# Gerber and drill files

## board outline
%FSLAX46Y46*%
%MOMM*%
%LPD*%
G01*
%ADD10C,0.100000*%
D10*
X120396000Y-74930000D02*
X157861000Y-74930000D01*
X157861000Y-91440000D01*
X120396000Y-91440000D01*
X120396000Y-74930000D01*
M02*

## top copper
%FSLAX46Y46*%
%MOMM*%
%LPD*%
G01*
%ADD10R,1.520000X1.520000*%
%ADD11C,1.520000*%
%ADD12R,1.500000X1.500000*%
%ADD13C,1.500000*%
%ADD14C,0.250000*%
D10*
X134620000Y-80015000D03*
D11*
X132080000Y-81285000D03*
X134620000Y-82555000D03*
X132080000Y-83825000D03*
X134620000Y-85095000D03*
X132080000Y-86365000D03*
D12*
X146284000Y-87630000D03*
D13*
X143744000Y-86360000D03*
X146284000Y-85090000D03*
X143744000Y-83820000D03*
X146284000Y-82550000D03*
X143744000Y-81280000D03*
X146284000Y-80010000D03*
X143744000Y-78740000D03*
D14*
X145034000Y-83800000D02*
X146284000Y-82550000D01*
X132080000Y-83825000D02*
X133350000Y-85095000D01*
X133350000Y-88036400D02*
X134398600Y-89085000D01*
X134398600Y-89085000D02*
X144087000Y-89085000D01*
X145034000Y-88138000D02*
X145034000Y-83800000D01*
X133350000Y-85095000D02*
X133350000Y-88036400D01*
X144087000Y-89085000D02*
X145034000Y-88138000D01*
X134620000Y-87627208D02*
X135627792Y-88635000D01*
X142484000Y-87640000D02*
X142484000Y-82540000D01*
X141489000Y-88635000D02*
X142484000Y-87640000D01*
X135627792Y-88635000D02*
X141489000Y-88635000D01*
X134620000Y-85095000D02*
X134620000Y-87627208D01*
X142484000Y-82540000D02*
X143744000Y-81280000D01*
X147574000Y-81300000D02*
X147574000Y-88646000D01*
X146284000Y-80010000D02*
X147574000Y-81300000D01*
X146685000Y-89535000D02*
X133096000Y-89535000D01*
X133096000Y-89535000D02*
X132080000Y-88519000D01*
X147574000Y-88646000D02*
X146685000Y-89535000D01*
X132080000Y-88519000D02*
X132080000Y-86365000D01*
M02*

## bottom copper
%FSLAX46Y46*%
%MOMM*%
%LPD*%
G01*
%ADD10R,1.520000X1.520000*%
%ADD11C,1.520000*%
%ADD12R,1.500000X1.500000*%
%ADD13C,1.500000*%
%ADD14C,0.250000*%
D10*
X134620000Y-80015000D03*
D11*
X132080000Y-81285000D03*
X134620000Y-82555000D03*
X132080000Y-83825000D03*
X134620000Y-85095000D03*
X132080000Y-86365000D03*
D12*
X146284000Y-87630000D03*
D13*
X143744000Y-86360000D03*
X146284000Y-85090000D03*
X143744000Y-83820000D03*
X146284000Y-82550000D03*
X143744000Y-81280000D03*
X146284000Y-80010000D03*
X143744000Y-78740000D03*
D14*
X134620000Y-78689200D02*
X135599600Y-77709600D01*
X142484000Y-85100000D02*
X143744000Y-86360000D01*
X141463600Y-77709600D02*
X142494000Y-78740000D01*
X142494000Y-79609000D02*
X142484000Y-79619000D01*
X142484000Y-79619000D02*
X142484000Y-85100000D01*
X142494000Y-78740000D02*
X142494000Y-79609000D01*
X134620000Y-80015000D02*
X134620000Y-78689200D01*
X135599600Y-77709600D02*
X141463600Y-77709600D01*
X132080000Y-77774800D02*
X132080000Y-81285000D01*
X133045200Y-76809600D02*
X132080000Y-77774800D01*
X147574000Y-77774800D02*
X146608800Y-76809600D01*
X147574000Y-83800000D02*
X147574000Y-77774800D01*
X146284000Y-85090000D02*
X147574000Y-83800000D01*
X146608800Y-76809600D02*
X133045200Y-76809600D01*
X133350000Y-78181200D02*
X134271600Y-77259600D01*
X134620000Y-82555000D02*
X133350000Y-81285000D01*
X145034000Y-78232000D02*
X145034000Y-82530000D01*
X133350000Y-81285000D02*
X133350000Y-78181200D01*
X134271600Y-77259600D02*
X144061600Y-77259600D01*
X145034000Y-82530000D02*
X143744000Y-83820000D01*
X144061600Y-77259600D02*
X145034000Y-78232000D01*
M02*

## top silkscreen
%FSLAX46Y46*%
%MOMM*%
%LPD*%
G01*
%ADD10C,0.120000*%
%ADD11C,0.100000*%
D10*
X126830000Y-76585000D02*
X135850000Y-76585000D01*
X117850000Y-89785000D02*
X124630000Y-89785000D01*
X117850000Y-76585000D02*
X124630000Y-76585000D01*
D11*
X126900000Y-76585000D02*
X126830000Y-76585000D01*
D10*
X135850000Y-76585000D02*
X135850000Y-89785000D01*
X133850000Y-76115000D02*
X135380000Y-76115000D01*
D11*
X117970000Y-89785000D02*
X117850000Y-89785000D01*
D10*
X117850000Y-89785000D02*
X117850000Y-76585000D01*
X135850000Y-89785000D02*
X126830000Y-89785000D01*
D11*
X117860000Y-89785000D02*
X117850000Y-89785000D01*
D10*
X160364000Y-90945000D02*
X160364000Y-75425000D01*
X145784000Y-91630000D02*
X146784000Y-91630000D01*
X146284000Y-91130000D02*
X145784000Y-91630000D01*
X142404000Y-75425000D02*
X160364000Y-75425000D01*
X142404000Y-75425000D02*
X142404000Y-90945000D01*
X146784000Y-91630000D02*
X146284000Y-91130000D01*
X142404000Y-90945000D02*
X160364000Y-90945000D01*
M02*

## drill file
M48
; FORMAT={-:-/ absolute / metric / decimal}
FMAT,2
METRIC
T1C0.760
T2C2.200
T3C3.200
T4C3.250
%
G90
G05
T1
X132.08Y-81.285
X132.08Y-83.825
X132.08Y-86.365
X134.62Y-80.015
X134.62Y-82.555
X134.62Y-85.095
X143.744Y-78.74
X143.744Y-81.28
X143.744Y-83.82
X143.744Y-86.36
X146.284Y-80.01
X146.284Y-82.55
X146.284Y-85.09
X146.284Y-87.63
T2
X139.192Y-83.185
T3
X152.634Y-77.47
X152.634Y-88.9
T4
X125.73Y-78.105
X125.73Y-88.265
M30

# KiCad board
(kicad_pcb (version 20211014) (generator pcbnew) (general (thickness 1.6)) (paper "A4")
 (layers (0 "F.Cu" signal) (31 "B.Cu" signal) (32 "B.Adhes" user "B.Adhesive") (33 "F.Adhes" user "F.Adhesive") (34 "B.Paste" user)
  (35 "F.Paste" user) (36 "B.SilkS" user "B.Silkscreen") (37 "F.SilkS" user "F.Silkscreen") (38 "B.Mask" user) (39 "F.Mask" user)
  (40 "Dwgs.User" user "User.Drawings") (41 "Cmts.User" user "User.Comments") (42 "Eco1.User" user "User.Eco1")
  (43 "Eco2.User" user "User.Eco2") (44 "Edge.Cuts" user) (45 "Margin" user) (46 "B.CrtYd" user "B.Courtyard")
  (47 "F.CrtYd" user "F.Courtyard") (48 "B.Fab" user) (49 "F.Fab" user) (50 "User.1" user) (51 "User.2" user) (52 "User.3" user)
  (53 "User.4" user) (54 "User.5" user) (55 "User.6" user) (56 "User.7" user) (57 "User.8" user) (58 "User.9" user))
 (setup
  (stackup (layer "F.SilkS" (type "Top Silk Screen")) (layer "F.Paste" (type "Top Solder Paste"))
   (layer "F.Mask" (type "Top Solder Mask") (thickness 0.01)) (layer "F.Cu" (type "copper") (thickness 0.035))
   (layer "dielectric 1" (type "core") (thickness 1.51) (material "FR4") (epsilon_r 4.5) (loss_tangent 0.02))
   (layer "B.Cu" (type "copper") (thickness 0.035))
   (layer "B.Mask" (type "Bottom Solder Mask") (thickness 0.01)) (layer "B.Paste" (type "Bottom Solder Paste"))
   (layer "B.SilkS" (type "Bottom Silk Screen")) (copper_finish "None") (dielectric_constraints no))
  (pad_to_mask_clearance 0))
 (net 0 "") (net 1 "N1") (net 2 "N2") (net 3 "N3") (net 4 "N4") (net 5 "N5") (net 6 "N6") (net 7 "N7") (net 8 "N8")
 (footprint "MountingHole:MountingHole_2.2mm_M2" (layer "F.Cu") (at 139.192 83.185)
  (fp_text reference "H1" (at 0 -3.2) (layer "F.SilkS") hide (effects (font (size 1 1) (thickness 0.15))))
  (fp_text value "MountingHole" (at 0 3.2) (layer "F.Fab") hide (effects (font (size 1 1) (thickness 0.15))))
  (pad "" np_thru_hole circle (at 0 0) (size 2.2 2.2) (drill 2.2) (layers *.Cu *.Mask)))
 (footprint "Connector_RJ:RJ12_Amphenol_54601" (layer "F.Cu") (at 134.62 80.015 -90)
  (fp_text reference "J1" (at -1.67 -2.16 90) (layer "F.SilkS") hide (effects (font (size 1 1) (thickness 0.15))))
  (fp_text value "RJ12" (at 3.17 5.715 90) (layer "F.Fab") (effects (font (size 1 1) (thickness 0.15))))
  (fp_line (start -3.43 7.79) (end -3.43 -1.23) (layer "F.SilkS") (width 0.12))
  (fp_line (start 9.77 16.77) (end 9.77 9.99) (layer "F.SilkS") (width 0.12))
  (fp_line (start -3.43 16.77) (end -3.43 9.99) (layer "F.SilkS") (width 0.12))
  (fp_line (start -3.43 7.72) (end -3.43 7.79) (layer "F.SilkS") (width 0.1))
  (fp_line (start -3.43 -1.23) (end 9.77 -1.23) (layer "F.SilkS") (width 0.12))
  (fp_line (start -3.9 0.77) (end -3.9 -0.76) (layer "F.SilkS") (width 0.12))
  (fp_line (start 9.77 16.65) (end 9.77 16.77) (layer "F.SilkS") (width 0.1))
  (fp_line (start 9.77 16.77) (end -3.43 16.77) (layer "F.SilkS") (width 0.12))
  (fp_line (start 9.77 -1.23) (end 9.77 7.79) (layer "F.SilkS") (width 0.12))
  (fp_line (start 9.77 16.76) (end 9.77 16.77) (layer "F.SilkS") (width 0.1))
  (pad "" np_thru_hole circle (at 8.25 8.89 270) (size 3.25 3.25) (drill 3.25) (layers *.Cu *.Mask))
  (pad "" np_thru_hole circle (at -1.91 8.89 270) (size 3.25 3.25) (drill 3.25) (layers *.Cu *.Mask))
  (pad "1" thru_hole rect (at 0 0 270) (size 1.52 1.52) (drill 0.76) (layers *.Cu *.Mask) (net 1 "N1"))
  (pad "2" thru_hole circle (at 1.27 2.54 270) (size 1.52 1.52) (drill 0.76) (layers *.Cu *.Mask) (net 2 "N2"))
  (pad "3" thru_hole circle (at 2.54 0 270) (size 1.52 1.52) (drill 0.76) (layers *.Cu *.Mask) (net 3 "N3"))
  (pad "4" thru_hole circle (at 3.81 2.54 270) (size 1.52 1.52) (drill 0.76) (layers *.Cu *.Mask) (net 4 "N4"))
  (pad "5" thru_hole circle (at 5.08 0 270) (size 1.52 1.52) (drill 0.76) (layers *.Cu *.Mask) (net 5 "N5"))
  (pad "6" thru_hole circle (at 6.35 2.54 270) (size 1.52 1.52) (drill 0.76) (layers *.Cu *.Mask) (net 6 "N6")))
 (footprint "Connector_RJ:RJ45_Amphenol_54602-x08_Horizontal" (layer "F.Cu") (at 146.284 87.63 90)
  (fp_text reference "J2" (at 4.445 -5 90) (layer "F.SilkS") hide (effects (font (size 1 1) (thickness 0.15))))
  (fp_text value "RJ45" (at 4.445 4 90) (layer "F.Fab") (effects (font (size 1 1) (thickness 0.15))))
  (fp_line (start -3.315 14.08) (end 12.205 14.08) (layer "F.SilkS") (width 0.12))
  (fp_line (start -4 -0.5) (end -4 0.5) (layer "F.SilkS") (width 0.12))
  (fp_line (start -3.5 0) (end -4 -0.5) (layer "F.SilkS") (width 0.12))
  (fp_line (start 12.205 -3.88) (end 12.205 14.08) (layer "F.SilkS") (width 0.12))
  (fp_line (start 12.205 -3.88) (end -3.315 -3.88) (layer "F.SilkS") (width 0.12))
  (fp_line (start -4 0.5) (end -3.5 0) (layer "F.SilkS") (width 0.12))
  (fp_line (start -3.315 -3.88) (end -3.315 14.08) (layer "F.SilkS") (width 0.12))
  (pad "" np_thru_hole circle (at 10.16 6.35 90) (size 3.2 3.2) (drill 3.2) (layers *.Cu *.Mask))
  (pad "" np_thru_hole circle (at -1.27 6.35 90) (size 3.2 3.2) (drill 3.2) (layers *.Cu *.Mask))
  (pad "1" thru_hole rect (at 0 0 90) (size 1.5 1.5) (drill 0.76) (layers *.Cu *.Mask) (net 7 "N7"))
  (pad "2" thru_hole circle (at 1.27 -2.54 90) (size 1.5 1.5) (drill 0.76) (layers *.Cu *.Mask) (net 1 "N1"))
  (pad "3" thru_hole circle (at 2.54 0 90) (size 1.5 1.5) (drill 0.76) (layers *.Cu *.Mask) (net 2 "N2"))
  (pad "4" thru_hole circle (at 3.81 -2.54 90) (size 1.5 1.5) (drill 0.76) (layers *.Cu *.Mask) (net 3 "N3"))
  (pad "5" thru_hole circle (at 5.08 0 90) (size 1.5 1.5) (drill 0.76) (layers *.Cu *.Mask) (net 4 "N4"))
  (pad "6" thru_hole circle (at 6.35 -2.54 90) (size 1.5 1.5) (drill 0.76) (layers *.Cu *.Mask) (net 5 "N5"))
  (pad "7" thru_hole circle (at 7.62 0 90) (size 1.5 1.5) (drill 0.76) (layers *.Cu *.Mask) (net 6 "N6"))
  (pad "8" thru_hole circle (at 8.89 -2.54 90) (size 1.5 1.5) (drill 0.76) (layers *.Cu *.Mask) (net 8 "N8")))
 (gr_rect (start 120.396 74.93) (end 157.861 91.44) (layer "Edge.Cuts") (width 0.1) (fill none))
 (segment (start 134.62 78.6892) (end 135.5996 77.7096) (width 0.25) (layer "B.Cu") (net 1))
 (segment (start 142.484 85.1) (end 143.744 86.36) (width 0.25) (layer "B.Cu") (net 1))
 (segment (start 141.4636 77.7096) (end 142.494 78.74) (width 0.25) (layer "B.Cu") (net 1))
 (segment (start 142.494 79.609) (end 142.484 79.619) (width 0.25) (layer "B.Cu") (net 1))
 (segment (start 142.484 79.619) (end 142.484 85.1) (width 0.25) (layer "B.Cu") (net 1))
 (segment (start 142.494 78.74) (end 142.494 79.609) (width 0.25) (layer "B.Cu") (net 1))
 (segment (start 134.62 80.015) (end 134.62 78.6892) (width 0.25) (layer "B.Cu") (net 1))
 (segment (start 135.5996 77.7096) (end 141.4636 77.7096) (width 0.25) (layer "B.Cu") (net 1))
 (segment (start 132.08 77.7748) (end 132.08 81.285) (width 0.25) (layer "B.Cu") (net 2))
 (segment (start 133.0452 76.8096) (end 132.08 77.7748) (width 0.25) (layer "B.Cu") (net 2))
 (segment (start 147.574 77.7748) (end 146.6088 76.8096) (width 0.25) (layer "B.Cu") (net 2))
 (segment (start 147.574 83.8) (end 147.574 77.7748) (width 0.25) (layer "B.Cu") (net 2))
 (segment (start 146.284 85.09) (end 147.574 83.8) (width 0.25) (layer "B.Cu") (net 2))
 (segment (start 146.6088 76.8096) (end 133.0452 76.8096) (width 0.25) (layer "B.Cu") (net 2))
 (segment (start 133.35 78.1812) (end 134.2716 77.2596) (width 0.25) (layer "B.Cu") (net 3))
 (segment (start 134.62 82.555) (end 133.35 81.285) (width 0.25) (layer "B.Cu") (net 3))
 (segment (start 145.034 78.232) (end 145.034 82.53) (width 0.25) (layer "B.Cu") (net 3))
 (segment (start 133.35 81.285) (end 133.35 78.1812) (width 0.25) (layer "B.Cu") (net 3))
 (segment (start 134.2716 77.2596) (end 144.0616 77.2596) (width 0.25) (layer "B.Cu") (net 3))
 (segment (start 145.034 82.53) (end 143.744 83.82) (width 0.25) (layer "B.Cu") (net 3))
 (segment (start 144.0616 77.2596) (end 145.034 78.232) (width 0.25) (layer "B.Cu") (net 3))
 (segment (start 145.034 83.8) (end 146.284 82.55) (width 0.25) (layer "F.Cu") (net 4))
 (segment (start 132.08 83.825) (end 133.35 85.095) (width 0.25) (layer "F.Cu") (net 4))
 (segment (start 133.35 88.0364) (end 134.3986 89.085) (width 0.25) (layer "F.Cu") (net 4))
 (segment (start 134.3986 89.085) (end 144.087 89.085) (width 0.25) (layer "F.Cu") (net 4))
 (segment (start 145.034 88.138) (end 145.034 83.8) (width 0.25) (layer "F.Cu") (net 4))
 (segment (start 133.35 85.095) (end 133.35 88.0364) (width 0.25) (layer "F.Cu") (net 4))
 (segment (start 144.087 89.085) (end 145.034 88.138) (width 0.25) (layer "F.Cu") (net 4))
 (segment (start 134.62 87.627208) (end 135.627792 88.635) (width 0.25) (layer "F.Cu") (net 5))
 (segment (start 142.484 87.64) (end 142.484 82.54) (width 0.25) (layer "F.Cu") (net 5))
 (segment (start 141.489 88.635) (end 142.484 87.64) (width 0.25) (layer "F.Cu") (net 5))
 (segment (start 135.627792 88.635) (end 141.489 88.635) (width 0.25) (layer "F.Cu") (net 5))
 (segment (start 134.62 85.095) (end 134.62 87.627208) (width 0.25) (layer "F.Cu") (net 5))
 (segment (start 142.484 82.54) (end 143.744 81.28) (width 0.25) (layer "F.Cu") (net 5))
 (segment (start 147.574 81.3) (end 147.574 88.646) (width 0.25) (layer "F.Cu") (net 6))
 (segment (start 146.284 80.01) (end 147.574 81.3) (width 0.25) (layer "F.Cu") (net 6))
 (segment (start 146.685 89.535) (end 133.096 89.535) (width 0.25) (layer "F.Cu") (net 6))
 (segment (start 133.096 89.535) (end 132.08 88.519) (width 0.25) (layer "F.Cu") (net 6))
 (segment (start 147.574 88.646) (end 146.685 89.535) (width 0.25) (layer "F.Cu") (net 6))
 (segment (start 132.08 88.519) (end 132.08 86.365) (width 0.25) (layer "F.Cu") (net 6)))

